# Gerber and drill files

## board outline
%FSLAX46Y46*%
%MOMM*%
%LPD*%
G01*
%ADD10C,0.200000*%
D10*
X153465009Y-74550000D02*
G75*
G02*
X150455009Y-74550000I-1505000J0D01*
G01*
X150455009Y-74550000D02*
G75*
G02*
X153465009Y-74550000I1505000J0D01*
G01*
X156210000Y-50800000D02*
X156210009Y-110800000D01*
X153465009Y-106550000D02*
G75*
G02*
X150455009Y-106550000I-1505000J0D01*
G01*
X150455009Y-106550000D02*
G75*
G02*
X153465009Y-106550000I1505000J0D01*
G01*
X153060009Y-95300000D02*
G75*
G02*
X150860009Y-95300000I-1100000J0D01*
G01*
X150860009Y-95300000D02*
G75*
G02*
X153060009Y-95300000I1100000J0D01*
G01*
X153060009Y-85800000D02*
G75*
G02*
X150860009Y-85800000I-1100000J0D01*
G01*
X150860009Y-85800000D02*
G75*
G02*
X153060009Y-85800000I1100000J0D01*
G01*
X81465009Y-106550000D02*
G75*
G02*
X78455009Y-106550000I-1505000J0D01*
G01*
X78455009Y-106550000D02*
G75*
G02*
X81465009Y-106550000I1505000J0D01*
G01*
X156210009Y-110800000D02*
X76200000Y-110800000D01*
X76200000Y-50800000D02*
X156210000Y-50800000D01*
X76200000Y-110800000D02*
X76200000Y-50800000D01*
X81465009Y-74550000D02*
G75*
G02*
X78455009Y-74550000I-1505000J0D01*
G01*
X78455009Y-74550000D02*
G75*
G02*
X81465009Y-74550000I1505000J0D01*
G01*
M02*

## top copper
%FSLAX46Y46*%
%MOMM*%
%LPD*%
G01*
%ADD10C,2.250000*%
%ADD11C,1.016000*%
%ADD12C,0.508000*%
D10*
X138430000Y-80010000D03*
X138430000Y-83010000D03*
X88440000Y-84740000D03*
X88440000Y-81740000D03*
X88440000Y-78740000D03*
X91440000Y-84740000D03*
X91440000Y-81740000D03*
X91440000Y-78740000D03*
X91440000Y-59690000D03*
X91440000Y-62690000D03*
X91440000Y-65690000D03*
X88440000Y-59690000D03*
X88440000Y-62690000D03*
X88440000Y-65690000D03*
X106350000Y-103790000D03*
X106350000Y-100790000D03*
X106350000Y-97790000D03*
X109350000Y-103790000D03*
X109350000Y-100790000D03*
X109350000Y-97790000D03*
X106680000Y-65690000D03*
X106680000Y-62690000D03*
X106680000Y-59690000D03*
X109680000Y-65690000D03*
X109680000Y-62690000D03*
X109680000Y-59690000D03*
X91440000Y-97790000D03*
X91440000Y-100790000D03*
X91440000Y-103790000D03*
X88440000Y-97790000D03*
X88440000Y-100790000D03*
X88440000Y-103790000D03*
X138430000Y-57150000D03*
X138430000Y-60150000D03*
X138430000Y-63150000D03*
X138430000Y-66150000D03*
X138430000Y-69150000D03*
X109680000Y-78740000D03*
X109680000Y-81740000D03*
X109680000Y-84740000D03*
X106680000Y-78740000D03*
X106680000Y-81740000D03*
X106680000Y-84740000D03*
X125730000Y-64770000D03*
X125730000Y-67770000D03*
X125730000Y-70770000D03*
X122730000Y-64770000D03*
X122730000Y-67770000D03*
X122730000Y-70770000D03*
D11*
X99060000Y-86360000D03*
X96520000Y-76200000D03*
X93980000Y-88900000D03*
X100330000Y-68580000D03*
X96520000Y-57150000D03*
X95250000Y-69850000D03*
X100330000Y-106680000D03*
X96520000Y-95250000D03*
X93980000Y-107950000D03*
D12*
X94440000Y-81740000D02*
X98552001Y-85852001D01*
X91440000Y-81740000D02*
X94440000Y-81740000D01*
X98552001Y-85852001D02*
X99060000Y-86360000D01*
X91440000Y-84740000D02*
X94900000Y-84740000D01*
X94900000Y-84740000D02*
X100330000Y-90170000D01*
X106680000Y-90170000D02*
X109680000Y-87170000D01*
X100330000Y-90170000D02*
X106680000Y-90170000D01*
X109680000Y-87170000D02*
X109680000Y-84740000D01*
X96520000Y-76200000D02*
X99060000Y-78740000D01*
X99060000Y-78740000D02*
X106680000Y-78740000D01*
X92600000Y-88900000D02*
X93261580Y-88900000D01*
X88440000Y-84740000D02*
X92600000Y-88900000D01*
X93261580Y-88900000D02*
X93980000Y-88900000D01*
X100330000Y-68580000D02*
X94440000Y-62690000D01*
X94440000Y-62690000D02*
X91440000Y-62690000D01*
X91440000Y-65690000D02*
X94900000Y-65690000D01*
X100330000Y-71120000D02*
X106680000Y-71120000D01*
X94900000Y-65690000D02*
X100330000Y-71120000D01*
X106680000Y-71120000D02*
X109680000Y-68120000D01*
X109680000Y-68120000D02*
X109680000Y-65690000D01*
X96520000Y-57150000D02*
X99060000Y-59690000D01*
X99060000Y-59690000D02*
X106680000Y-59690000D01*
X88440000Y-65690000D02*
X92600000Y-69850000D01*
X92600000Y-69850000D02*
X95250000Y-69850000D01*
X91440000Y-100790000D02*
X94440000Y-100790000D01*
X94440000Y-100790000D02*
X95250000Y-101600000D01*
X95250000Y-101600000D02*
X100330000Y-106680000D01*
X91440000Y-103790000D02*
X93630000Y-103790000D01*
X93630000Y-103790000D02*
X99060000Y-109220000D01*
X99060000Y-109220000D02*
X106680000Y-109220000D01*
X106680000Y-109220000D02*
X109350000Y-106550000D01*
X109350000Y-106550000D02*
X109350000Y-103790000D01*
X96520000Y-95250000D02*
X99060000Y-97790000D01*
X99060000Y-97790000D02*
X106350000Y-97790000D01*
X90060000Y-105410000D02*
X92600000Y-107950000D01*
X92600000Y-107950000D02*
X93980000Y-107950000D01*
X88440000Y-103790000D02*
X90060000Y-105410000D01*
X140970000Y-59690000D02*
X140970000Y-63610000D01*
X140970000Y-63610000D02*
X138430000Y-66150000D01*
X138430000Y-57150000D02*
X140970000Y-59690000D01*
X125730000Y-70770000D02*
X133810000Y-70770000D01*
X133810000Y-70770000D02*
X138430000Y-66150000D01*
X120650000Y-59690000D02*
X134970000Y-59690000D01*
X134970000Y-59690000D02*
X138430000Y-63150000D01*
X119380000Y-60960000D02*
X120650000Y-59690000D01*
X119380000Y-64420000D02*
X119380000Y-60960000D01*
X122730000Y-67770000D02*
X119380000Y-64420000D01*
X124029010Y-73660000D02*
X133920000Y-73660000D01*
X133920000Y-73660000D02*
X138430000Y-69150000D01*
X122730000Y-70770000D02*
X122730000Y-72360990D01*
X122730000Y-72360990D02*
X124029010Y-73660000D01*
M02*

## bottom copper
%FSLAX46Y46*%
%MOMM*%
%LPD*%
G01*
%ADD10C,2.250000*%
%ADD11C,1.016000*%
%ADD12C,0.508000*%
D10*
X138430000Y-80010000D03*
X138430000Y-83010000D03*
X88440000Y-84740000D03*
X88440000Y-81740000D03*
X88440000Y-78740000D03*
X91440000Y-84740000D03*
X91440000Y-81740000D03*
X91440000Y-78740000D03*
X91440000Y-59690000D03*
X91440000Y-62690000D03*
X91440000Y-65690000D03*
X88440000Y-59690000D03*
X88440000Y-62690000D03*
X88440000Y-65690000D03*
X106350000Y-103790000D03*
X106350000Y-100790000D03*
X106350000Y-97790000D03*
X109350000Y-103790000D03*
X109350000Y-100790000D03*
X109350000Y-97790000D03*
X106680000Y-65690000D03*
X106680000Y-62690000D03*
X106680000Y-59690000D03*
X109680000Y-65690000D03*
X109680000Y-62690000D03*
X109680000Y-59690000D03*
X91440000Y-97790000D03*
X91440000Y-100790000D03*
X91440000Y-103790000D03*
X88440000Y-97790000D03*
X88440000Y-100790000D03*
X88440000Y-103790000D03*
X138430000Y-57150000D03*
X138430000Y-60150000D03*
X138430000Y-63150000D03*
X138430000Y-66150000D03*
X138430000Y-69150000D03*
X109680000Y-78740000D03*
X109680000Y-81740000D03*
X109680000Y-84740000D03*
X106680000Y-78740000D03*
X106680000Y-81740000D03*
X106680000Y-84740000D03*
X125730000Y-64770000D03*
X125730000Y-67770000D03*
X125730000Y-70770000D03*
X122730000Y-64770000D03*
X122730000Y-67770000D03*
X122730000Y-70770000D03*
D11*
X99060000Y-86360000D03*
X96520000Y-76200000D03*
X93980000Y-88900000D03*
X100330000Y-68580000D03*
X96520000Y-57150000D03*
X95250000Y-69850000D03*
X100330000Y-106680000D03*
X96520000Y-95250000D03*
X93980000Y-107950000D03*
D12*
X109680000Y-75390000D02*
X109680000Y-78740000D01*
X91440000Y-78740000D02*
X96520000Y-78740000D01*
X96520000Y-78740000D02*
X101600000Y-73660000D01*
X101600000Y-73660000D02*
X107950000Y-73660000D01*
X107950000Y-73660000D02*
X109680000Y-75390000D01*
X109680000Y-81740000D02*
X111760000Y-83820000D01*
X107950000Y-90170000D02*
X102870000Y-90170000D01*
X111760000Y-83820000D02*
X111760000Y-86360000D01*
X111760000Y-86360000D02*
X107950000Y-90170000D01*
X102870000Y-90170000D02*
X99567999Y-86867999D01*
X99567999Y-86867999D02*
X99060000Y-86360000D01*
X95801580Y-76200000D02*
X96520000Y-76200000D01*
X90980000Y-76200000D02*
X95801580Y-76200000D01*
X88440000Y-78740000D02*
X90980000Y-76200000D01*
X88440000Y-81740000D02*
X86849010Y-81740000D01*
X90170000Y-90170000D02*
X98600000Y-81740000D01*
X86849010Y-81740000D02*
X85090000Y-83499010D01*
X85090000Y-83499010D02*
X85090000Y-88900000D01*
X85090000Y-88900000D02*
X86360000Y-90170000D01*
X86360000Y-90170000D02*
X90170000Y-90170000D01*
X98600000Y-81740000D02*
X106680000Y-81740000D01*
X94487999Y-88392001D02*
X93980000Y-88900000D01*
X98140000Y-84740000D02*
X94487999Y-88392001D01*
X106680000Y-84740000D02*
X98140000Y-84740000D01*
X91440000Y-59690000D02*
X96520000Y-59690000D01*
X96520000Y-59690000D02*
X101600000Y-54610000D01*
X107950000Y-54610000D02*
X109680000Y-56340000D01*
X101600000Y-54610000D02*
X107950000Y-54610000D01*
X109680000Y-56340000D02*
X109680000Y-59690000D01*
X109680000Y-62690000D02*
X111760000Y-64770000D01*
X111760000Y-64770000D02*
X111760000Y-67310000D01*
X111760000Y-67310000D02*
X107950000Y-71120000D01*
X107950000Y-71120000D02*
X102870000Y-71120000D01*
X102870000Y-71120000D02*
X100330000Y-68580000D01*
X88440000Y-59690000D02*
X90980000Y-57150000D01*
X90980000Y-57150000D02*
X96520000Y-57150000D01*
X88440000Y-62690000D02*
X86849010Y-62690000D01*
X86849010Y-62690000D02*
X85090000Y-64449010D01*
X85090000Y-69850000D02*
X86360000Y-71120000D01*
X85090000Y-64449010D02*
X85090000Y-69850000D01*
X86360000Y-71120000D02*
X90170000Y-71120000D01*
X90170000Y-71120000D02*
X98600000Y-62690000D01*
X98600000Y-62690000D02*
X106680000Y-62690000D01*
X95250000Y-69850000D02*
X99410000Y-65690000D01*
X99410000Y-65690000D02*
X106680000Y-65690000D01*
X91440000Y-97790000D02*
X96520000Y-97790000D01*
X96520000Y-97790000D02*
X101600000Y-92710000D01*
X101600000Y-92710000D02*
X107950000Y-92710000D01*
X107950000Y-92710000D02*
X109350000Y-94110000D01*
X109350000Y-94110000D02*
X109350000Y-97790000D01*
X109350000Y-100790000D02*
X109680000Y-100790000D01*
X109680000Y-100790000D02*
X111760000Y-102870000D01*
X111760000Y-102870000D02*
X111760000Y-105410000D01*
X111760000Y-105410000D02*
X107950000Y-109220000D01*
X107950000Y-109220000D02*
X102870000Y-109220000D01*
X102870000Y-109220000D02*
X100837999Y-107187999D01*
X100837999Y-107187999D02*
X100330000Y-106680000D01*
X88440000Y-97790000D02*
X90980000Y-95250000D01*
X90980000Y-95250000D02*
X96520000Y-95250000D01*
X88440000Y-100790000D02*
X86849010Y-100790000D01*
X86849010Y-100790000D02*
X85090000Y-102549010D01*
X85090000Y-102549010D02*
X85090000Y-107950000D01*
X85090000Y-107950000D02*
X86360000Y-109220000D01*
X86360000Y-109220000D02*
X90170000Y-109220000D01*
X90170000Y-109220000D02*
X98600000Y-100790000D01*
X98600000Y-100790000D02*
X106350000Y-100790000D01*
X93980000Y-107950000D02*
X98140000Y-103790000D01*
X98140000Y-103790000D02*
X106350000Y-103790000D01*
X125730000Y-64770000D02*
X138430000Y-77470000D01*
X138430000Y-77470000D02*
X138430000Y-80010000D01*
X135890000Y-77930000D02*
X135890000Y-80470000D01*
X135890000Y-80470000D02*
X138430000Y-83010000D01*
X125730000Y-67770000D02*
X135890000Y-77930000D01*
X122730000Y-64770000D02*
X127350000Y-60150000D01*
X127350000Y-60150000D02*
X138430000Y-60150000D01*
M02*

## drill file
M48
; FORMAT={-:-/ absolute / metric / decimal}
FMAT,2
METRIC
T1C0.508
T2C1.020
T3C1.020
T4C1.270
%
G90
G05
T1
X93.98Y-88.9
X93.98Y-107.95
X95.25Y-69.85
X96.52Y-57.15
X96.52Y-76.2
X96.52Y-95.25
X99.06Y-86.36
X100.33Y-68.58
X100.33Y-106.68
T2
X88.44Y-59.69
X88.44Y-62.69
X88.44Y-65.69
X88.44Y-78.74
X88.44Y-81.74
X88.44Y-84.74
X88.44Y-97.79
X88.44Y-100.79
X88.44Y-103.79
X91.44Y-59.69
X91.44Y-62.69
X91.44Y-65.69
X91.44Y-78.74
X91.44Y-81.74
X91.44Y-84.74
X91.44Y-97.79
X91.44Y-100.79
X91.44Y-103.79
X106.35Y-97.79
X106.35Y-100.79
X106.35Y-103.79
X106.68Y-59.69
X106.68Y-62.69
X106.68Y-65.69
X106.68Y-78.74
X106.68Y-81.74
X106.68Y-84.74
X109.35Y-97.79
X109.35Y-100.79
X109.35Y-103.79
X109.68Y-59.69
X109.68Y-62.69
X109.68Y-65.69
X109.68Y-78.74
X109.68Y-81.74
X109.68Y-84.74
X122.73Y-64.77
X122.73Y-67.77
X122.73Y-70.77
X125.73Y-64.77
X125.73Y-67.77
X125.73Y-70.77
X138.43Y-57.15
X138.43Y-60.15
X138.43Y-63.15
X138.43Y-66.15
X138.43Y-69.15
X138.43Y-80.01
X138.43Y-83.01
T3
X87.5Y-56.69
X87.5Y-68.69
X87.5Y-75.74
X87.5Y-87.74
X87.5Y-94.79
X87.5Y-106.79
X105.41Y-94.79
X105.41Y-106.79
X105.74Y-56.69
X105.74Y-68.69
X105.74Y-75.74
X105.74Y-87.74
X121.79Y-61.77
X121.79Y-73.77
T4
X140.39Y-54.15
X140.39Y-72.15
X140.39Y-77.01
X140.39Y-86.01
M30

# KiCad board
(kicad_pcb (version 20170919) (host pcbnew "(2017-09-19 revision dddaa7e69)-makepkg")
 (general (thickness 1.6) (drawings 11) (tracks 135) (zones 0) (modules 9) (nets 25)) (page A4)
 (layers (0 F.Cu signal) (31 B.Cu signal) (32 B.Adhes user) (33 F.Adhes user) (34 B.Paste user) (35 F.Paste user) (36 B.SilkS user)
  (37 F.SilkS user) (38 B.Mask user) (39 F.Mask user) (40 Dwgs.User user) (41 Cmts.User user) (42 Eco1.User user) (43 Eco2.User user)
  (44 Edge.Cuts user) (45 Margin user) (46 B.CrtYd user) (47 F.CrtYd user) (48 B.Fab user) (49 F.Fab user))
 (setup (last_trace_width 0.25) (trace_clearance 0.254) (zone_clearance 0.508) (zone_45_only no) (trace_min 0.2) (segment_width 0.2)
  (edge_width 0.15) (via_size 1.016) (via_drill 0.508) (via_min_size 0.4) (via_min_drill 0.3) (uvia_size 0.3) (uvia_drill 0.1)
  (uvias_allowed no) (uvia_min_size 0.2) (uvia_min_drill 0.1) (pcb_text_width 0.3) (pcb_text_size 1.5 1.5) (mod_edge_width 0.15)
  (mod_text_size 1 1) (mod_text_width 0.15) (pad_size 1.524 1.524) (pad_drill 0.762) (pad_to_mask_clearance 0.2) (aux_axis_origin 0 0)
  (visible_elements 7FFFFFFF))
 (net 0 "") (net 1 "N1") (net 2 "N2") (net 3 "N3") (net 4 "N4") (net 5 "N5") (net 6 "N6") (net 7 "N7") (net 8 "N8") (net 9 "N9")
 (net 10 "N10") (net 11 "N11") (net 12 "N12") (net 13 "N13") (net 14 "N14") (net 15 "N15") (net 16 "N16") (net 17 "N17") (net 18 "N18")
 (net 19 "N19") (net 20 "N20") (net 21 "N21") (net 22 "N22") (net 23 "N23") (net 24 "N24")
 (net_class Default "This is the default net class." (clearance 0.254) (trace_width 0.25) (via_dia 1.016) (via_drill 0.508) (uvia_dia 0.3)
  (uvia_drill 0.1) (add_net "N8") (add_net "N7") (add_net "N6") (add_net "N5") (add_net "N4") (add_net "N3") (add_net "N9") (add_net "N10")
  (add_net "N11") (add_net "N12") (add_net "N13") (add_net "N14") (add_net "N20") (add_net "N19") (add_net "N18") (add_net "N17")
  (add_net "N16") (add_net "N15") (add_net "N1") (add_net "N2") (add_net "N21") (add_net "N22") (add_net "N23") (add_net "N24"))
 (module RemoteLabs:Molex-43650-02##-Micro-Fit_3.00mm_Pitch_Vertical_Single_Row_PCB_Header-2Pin (layer F.Cu) (at 138.43 80.01 90)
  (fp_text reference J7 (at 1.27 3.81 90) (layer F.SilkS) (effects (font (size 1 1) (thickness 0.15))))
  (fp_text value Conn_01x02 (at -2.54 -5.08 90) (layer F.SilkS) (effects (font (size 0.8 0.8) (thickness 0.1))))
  (pad 1 thru_hole circle (at 0 0 90) (size 2.25 2.25) (drill 1.02) (layers *.Cu *.Mask F.SilkS) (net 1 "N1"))
  (pad 2 thru_hole circle (at -3 0 90) (size 2.25 2.25) (drill 1.02) (layers *.Cu *.Mask F.SilkS) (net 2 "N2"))
  (pad "" np_thru_hole circle (at 3 1.96 90) (size 1.27 1.27) (drill 1.27) (layers *.Cu *.Mask F.SilkS))
  (pad "" np_thru_hole circle (at -6 1.96 90) (size 1.27 1.27) (drill 1.27) (layers *.Cu *.Mask F.SilkS)))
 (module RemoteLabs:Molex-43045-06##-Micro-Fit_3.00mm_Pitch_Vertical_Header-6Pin (layer F.Cu) (at 91.44 78.74 90)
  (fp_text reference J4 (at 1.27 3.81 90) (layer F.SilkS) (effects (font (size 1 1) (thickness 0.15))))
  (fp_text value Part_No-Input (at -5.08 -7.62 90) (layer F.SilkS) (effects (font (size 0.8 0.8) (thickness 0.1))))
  (pad 6 thru_hole circle (at -6 -3 90) (size 2.25 2.25) (drill 1.02) (layers *.Cu *.Mask F.SilkS) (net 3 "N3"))
  (pad 5 thru_hole circle (at -3 -3 90) (size 2.25 2.25) (drill 1.02) (layers *.Cu *.Mask F.SilkS) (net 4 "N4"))
  (pad 4 thru_hole circle (at 0 -3 90) (size 2.25 2.25) (drill 1.02) (layers *.Cu *.Mask F.SilkS) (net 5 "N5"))
  (pad 3 thru_hole circle (at -6 0 90) (size 2.25 2.25) (drill 1.02) (layers *.Cu *.Mask F.SilkS) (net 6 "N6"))
  (pad 2 thru_hole circle (at -3 0 90) (size 2.25 2.25) (drill 1.02) (layers *.Cu *.Mask F.SilkS) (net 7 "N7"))
  (pad 1 thru_hole circle (at 0 0 90) (size 2.25 2.25) (drill 1.02) (layers *.Cu *.Mask F.SilkS) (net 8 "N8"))
  (pad "" np_thru_hole circle (at -9 -3.94 90) (size 1.02 1.02) (drill 1.02) (layers *.Cu *.Mask F.SilkS))
  (pad "" np_thru_hole circle (at 3 -3.94 90) (size 1.02 1.02) (drill 1.02) (layers *.Cu *.Mask F.SilkS)))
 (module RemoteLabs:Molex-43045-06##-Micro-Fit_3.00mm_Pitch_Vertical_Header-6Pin (layer F.Cu) (at 91.44 59.69 90)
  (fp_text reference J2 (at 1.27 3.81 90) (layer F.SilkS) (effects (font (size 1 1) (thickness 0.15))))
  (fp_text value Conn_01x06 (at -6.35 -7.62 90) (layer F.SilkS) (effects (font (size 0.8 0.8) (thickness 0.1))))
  (pad "" np_thru_hole circle (at 3 -3.94 90) (size 1.02 1.02) (drill 1.02) (layers *.Cu *.Mask F.SilkS))
  (pad "" np_thru_hole circle (at -9 -3.94 90) (size 1.02 1.02) (drill 1.02) (layers *.Cu *.Mask F.SilkS))
  (pad 1 thru_hole circle (at 0 0 90) (size 2.25 2.25) (drill 1.02) (layers *.Cu *.Mask F.SilkS) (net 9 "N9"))
  (pad 2 thru_hole circle (at -3 0 90) (size 2.25 2.25) (drill 1.02) (layers *.Cu *.Mask F.SilkS) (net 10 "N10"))
  (pad 3 thru_hole circle (at -6 0 90) (size 2.25 2.25) (drill 1.02) (layers *.Cu *.Mask F.SilkS) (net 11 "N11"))
  (pad 4 thru_hole circle (at 0 -3 90) (size 2.25 2.25) (drill 1.02) (layers *.Cu *.Mask F.SilkS) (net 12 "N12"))
  (pad 5 thru_hole circle (at -3 -3 90) (size 2.25 2.25) (drill 1.02) (layers *.Cu *.Mask F.SilkS) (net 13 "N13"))
  (pad 6 thru_hole circle (at -6 -3 90) (size 2.25 2.25) (drill 1.02) (layers *.Cu *.Mask F.SilkS) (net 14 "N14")))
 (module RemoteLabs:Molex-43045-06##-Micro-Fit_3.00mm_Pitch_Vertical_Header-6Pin (layer F.Cu) (at 109.35 97.79 90)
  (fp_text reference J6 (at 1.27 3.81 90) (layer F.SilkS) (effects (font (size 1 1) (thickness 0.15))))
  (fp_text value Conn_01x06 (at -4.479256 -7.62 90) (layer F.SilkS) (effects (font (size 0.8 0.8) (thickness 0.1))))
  (pad 6 thru_hole circle (at -6 -3 90) (size 2.25 2.25) (drill 1.02) (layers *.Cu *.Mask F.SilkS) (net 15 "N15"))
  (pad 5 thru_hole circle (at -3 -3 90) (size 2.25 2.25) (drill 1.02) (layers *.Cu *.Mask F.SilkS) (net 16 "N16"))
  (pad 4 thru_hole circle (at 0 -3 90) (size 2.25 2.25) (drill 1.02) (layers *.Cu *.Mask F.SilkS) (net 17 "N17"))
  (pad 3 thru_hole circle (at -6 0 90) (size 2.25 2.25) (drill 1.02) (layers *.Cu *.Mask F.SilkS) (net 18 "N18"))
  (pad 2 thru_hole circle (at -3 0 90) (size 2.25 2.25) (drill 1.02) (layers *.Cu *.Mask F.SilkS) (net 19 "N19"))
  (pad 1 thru_hole circle (at 0 0 90) (size 2.25 2.25) (drill 1.02) (layers *.Cu *.Mask F.SilkS) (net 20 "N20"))
  (pad "" np_thru_hole circle (at -9 -3.94 90) (size 1.02 1.02) (drill 1.02) (layers *.Cu *.Mask F.SilkS))
  (pad "" np_thru_hole circle (at 3 -3.94 90) (size 1.02 1.02) (drill 1.02) (layers *.Cu *.Mask F.SilkS)))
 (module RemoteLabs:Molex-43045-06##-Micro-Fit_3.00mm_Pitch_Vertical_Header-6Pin (layer F.Cu) (at 109.68 59.69 90)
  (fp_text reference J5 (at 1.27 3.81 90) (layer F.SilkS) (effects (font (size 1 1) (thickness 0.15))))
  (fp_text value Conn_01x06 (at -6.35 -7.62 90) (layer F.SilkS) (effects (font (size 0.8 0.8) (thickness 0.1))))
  (pad 6 thru_hole circle (at -6 -3 90) (size 2.25 2.25) (drill 1.02) (layers *.Cu *.Mask F.SilkS) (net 14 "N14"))
  (pad 5 thru_hole circle (at -3 -3 90) (size 2.25 2.25) (drill 1.02) (layers *.Cu *.Mask F.SilkS) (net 13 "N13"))
  (pad 4 thru_hole circle (at 0 -3 90) (size 2.25 2.25) (drill 1.02) (layers *.Cu *.Mask F.SilkS) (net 12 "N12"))
  (pad 3 thru_hole circle (at -6 0 90) (size 2.25 2.25) (drill 1.02) (layers *.Cu *.Mask F.SilkS) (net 11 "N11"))
  (pad 2 thru_hole circle (at -3 0 90) (size 2.25 2.25) (drill 1.02) (layers *.Cu *.Mask F.SilkS) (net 10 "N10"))
  (pad 1 thru_hole circle (at 0 0 90) (size 2.25 2.25) (drill 1.02) (layers *.Cu *.Mask F.SilkS) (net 9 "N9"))
  (pad "" np_thru_hole circle (at -9 -3.94 90) (size 1.02 1.02) (drill 1.02) (layers *.Cu *.Mask F.SilkS))
  (pad "" np_thru_hole circle (at 3 -3.94 90) (size 1.02 1.02) (drill 1.02) (layers *.Cu *.Mask F.SilkS)))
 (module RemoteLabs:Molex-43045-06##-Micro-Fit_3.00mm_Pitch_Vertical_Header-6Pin (layer F.Cu) (at 91.44 97.79 90)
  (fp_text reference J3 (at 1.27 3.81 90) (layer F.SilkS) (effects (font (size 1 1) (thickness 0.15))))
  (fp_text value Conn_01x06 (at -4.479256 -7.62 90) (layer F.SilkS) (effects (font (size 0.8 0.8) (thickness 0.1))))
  (pad "" np_thru_hole circle (at 3 -3.94 90) (size 1.02 1.02) (drill 1.02) (layers *.Cu *.Mask F.SilkS))
  (pad "" np_thru_hole circle (at -9 -3.94 90) (size 1.02 1.02) (drill 1.02) (layers *.Cu *.Mask F.SilkS))
  (pad 1 thru_hole circle (at 0 0 90) (size 2.25 2.25) (drill 1.02) (layers *.Cu *.Mask F.SilkS) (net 20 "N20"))
  (pad 2 thru_hole circle (at -3 0 90) (size 2.25 2.25) (drill 1.02) (layers *.Cu *.Mask F.SilkS) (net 19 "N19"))
  (pad 3 thru_hole circle (at -6 0 90) (size 2.25 2.25) (drill 1.02) (layers *.Cu *.Mask F.SilkS) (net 18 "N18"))
  (pad 4 thru_hole circle (at 0 -3 90) (size 2.25 2.25) (drill 1.02) (layers *.Cu *.Mask F.SilkS) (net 17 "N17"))
  (pad 5 thru_hole circle (at -3 -3 90) (size 2.25 2.25) (drill 1.02) (layers *.Cu *.Mask F.SilkS) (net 16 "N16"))
  (pad 6 thru_hole circle (at -6 -3 90) (size 2.25 2.25) (drill 1.02) (layers *.Cu *.Mask F.SilkS) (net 15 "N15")))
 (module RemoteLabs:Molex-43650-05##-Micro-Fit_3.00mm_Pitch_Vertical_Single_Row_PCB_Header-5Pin (layer F.Cu) (at 138.43 57.15 90)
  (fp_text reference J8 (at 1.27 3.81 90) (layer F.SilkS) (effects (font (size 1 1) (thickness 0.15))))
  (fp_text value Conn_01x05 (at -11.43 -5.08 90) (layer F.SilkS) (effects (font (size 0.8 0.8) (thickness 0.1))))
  (pad 1 thru_hole circle (at 0 0 90) (size 2.25 2.25) (drill 1.02) (layers *.Cu *.Mask F.SilkS) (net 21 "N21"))
  (pad 2 thru_hole circle (at -3 0 90) (size 2.25 2.25) (drill 1.02) (layers *.Cu *.Mask F.SilkS) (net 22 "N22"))
  (pad 3 thru_hole circle (at -6 0 90) (size 2.25 2.25) (drill 1.02) (layers *.Cu *.Mask F.SilkS) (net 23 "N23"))
  (pad 4 thru_hole circle (at -9 0 90) (size 2.25 2.25) (drill 1.02) (layers *.Cu *.Mask F.SilkS) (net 21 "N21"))
  (pad 5 thru_hole circle (at -12 0 90) (size 2.25 2.25) (drill 1.02) (layers *.Cu *.Mask F.SilkS) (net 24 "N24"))
  (pad "" np_thru_hole circle (at 3 1.96 90) (size 1.27 1.27) (drill 1.27) (layers *.Cu *.Mask F.SilkS))
  (pad "" np_thru_hole circle (at -15 1.96 90) (size 1.27 1.27) (drill 1.27) (layers *.Cu *.Mask F.SilkS)))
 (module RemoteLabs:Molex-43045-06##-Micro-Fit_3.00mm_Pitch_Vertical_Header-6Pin (layer F.Cu) (at 109.68 78.74 90)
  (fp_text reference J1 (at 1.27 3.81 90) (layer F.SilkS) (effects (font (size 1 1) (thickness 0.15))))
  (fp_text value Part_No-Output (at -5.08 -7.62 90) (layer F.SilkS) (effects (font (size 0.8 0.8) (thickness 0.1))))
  (pad "" np_thru_hole circle (at 3 -3.94 90) (size 1.02 1.02) (drill 1.02) (layers *.Cu *.Mask F.SilkS))
  (pad "" np_thru_hole circle (at -9 -3.94 90) (size 1.02 1.02) (drill 1.02) (layers *.Cu *.Mask F.SilkS))
  (pad 1 thru_hole circle (at 0 0 90) (size 2.25 2.25) (drill 1.02) (layers *.Cu *.Mask F.SilkS) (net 8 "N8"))
  (pad 2 thru_hole circle (at -3 0 90) (size 2.25 2.25) (drill 1.02) (layers *.Cu *.Mask F.SilkS) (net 7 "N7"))
  (pad 3 thru_hole circle (at -6 0 90) (size 2.25 2.25) (drill 1.02) (layers *.Cu *.Mask F.SilkS) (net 6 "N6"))
  (pad 4 thru_hole circle (at 0 -3 90) (size 2.25 2.25) (drill 1.02) (layers *.Cu *.Mask F.SilkS) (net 5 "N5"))
  (pad 5 thru_hole circle (at -3 -3 90) (size 2.25 2.25) (drill 1.02) (layers *.Cu *.Mask F.SilkS) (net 4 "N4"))
  (pad 6 thru_hole circle (at -6 -3 90) (size 2.25 2.25) (drill 1.02) (layers *.Cu *.Mask F.SilkS) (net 3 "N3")))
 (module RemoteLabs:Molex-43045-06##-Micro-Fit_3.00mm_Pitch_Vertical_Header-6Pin (layer F.Cu) (at 125.73 64.77 90)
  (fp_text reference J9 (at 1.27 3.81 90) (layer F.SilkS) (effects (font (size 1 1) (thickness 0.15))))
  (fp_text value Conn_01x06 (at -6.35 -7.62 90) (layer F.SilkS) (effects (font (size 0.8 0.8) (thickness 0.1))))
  (pad "" np_thru_hole circle (at 3 -3.94 90) (size 1.02 1.02) (drill 1.02) (layers *.Cu *.Mask F.SilkS))
  (pad "" np_thru_hole circle (at -9 -3.94 90) (size 1.02 1.02) (drill 1.02) (layers *.Cu *.Mask F.SilkS))
  (pad 1 thru_hole circle (at 0 0 90) (size 2.25 2.25) (drill 1.02) (layers *.Cu *.Mask F.SilkS) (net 1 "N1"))
  (pad 2 thru_hole circle (at -3 0 90) (size 2.25 2.25) (drill 1.02) (layers *.Cu *.Mask F.SilkS) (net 2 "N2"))
  (pad 3 thru_hole circle (at -6 0 90) (size 2.25 2.25) (drill 1.02) (layers *.Cu *.Mask F.SilkS) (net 21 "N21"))
  (pad 4 thru_hole circle (at 0 -3 90) (size 2.25 2.25) (drill 1.02) (layers *.Cu *.Mask F.SilkS) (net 22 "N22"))
  (pad 5 thru_hole circle (at -3 -3 90) (size 2.25 2.25) (drill 1.02) (layers *.Cu *.Mask F.SilkS) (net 23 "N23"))
  (pad 6 thru_hole circle (at -6 -3 90) (size 2.25 2.25) (drill 1.02) (layers *.Cu *.Mask F.SilkS) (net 24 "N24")))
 (gr_circle (center 151.960009 74.55) (end 153.465009 74.55) (layer Edge.Cuts) (width 0.2))
 (gr_line (start 156.21 50.8) (end 156.210009 110.8) (layer Edge.Cuts) (width 0.2))
 (gr_circle (center 151.960009 106.55) (end 153.465009 106.55) (layer Edge.Cuts) (width 0.2))
 (gr_circle (center 151.960009 95.3) (end 153.060009 95.3) (layer Edge.Cuts) (width 0.2))
 (gr_circle (center 151.960009 85.8) (end 153.060009 85.8) (layer Edge.Cuts) (width 0.2))
 (gr_circle (center 79.960009 106.55) (end 81.465009 106.55) (layer Edge.Cuts) (width 0.2))
 (gr_line (start 156.210009 110.8) (end 76.2 110.8) (layer Edge.Cuts) (width 0.2))
 (gr_line (start 76.2 50.8) (end 156.21 50.8) (layer Edge.Cuts) (width 0.2))
 (gr_line (start 76.2 110.8) (end 76.2 50.8) (layer Edge.Cuts) (width 0.2))
 (gr_circle (center 79.960009 74.55) (end 81.465009 74.55) (layer Edge.Cuts) (width 0.2))
 (segment (start 109.68 75.39) (end 109.68 78.74) (width 0.508) (layer B.Cu) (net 8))
 (segment (start 91.44 78.74) (end 96.52 78.74) (width 0.508) (layer B.Cu) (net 8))
 (segment (start 96.52 78.74) (end 101.6 73.66) (width 0.508) (layer B.Cu) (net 8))
 (segment (start 101.6 73.66) (end 107.95 73.66) (width 0.508) (layer B.Cu) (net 8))
 (segment (start 107.95 73.66) (end 109.68 75.39) (width 0.508) (layer B.Cu) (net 8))
 (segment (start 109.68 81.74) (end 111.76 83.82) (width 0.508) (layer B.Cu) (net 7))
 (segment (start 107.95 90.17) (end 102.87 90.17) (width 0.508) (layer B.Cu) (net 7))
 (segment (start 111.76 83.82) (end 111.76 86.36) (width 0.508) (layer B.Cu) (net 7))
 (segment (start 111.76 86.36) (end 107.95 90.17) (width 0.508) (layer B.Cu) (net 7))
 (segment (start 102.87 90.17) (end 99.567999 86.867999) (width 0.508) (layer B.Cu) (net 7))
 (segment (start 99.567999 86.867999) (end 99.06 86.36) (width 0.508) (layer B.Cu) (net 7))
 (segment (start 94.44 81.74) (end 98.552001 85.852001) (width 0.508) (layer F.Cu) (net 7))
 (segment (start 91.44 81.74) (end 94.44 81.74) (width 0.508) (layer F.Cu) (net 7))
 (segment (start 98.552001 85.852001) (end 99.06 86.36) (width 0.508) (layer F.Cu) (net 7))
 (via (at 99.06 86.36) (size 1.016) (drill 0.508) (layers F.Cu B.Cu) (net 7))
 (segment (start 91.44 84.74) (end 94.9 84.74) (width 0.508) (layer F.Cu) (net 6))
 (segment (start 94.9 84.74) (end 100.33 90.17) (width 0.508) (layer F.Cu) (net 6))
 (segment (start 106.68 90.17) (end 109.68 87.17) (width 0.508) (layer F.Cu) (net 6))
 (segment (start 100.33 90.17) (end 106.68 90.17) (width 0.508) (layer F.Cu) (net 6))
 (segment (start 109.68 87.17) (end 109.68 84.74) (width 0.508) (layer F.Cu) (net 6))
 (segment (start 96.52 76.2) (end 99.06 78.74) (width 0.508) (layer F.Cu) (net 5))
 (segment (start 99.06 78.74) (end 106.68 78.74) (width 0.508) (layer F.Cu) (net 5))
 (segment (start 95.80158 76.2) (end 96.52 76.2) (width 0.508) (layer B.Cu) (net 5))
 (segment (start 90.98 76.2) (end 95.80158 76.2) (width 0.508) (layer B.Cu) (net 5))
 (segment (start 88.44 78.74) (end 90.98 76.2) (width 0.508) (layer B.Cu) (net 5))
 (via (at 96.52 76.2) (size 1.016) (drill 0.508) (layers F.Cu B.Cu) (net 5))
 (segment (start 88.44 81.74) (end 86.84901 81.74) (width 0.508) (layer B.Cu) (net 4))
 (segment (start 90.17 90.17) (end 98.6 81.74) (width 0.508) (layer B.Cu) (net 4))
 (segment (start 86.84901 81.74) (end 85.09 83.49901) (width 0.508) (layer B.Cu) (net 4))
 (segment (start 85.09 83.49901) (end 85.09 88.9) (width 0.508) (layer B.Cu) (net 4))
 (segment (start 85.09 88.9) (end 86.36 90.17) (width 0.508) (layer B.Cu) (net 4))
 (segment (start 86.36 90.17) (end 90.17 90.17) (width 0.508) (layer B.Cu) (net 4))
 (segment (start 98.6 81.74) (end 106.68 81.74) (width 0.508) (layer B.Cu) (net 4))
 (segment (start 92.6 88.9) (end 93.26158 88.9) (width 0.508) (layer F.Cu) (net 3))
 (segment (start 88.44 84.74) (end 92.6 88.9) (width 0.508) (layer F.Cu) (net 3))
 (segment (start 93.26158 88.9) (end 93.98 88.9) (width 0.508) (layer F.Cu) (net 3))
 (segment (start 94.487999 88.392001) (end 93.98 88.9) (width 0.508) (layer B.Cu) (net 3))
 (segment (start 98.14 84.74) (end 94.487999 88.392001) (width 0.508) (layer B.Cu) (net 3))
 (segment (start 106.68 84.74) (end 98.14 84.74) (width 0.508) (layer B.Cu) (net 3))
 (via (at 93.98 88.9) (size 1.016) (drill 0.508) (layers F.Cu B.Cu) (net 3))
 (segment (start 91.44 59.69) (end 96.52 59.69) (width 0.508) (layer B.Cu) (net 9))
 (segment (start 96.52 59.69) (end 101.6 54.61) (width 0.508) (layer B.Cu) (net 9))
 (segment (start 107.95 54.61) (end 109.68 56.34) (width 0.508) (layer B.Cu) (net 9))
 (segment (start 101.6 54.61) (end 107.95 54.61) (width 0.508) (layer B.Cu) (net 9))
 (segment (start 109.68 56.34) (end 109.68 59.69) (width 0.508) (layer B.Cu) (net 9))
 (segment (start 109.68 62.69) (end 111.76 64.77) (width 0.508) (layer B.Cu) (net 10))
 (segment (start 111.76 64.77) (end 111.76 67.31) (width 0.508) (layer B.Cu) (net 10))
 (segment (start 111.76 67.31) (end 107.95 71.12) (width 0.508) (layer B.Cu) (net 10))
 (segment (start 107.95 71.12) (end 102.87 71.12) (width 0.508) (layer B.Cu) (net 10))
 (segment (start 102.87 71.12) (end 100.33 68.58) (width 0.508) (layer B.Cu) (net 10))
 (segment (start 100.33 68.58) (end 94.44 62.69) (width 0.508) (layer F.Cu) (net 10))
 (segment (start 94.44 62.69) (end 91.44 62.69) (width 0.508) (layer F.Cu) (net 10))
 (via (at 100.33 68.58) (size 1.016) (drill 0.508) (layers F.Cu B.Cu) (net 10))
 (segment (start 91.44 65.69) (end 94.9 65.69) (width 0.508) (layer F.Cu) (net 11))
 (segment (start 100.33 71.12) (end 106.68 71.12) (width 0.508) (layer F.Cu) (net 11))
 (segment (start 94.9 65.69) (end 100.33 71.12) (width 0.508) (layer F.Cu) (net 11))
 (segment (start 106.68 71.12) (end 109.68 68.12) (width 0.508) (layer F.Cu) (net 11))
 (segment (start 109.68 68.12) (end 109.68 65.69) (width 0.508) (layer F.Cu) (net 11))
 (segment (start 96.52 57.15) (end 99.06 59.69) (width 0.508) (layer F.Cu) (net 12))
 (segment (start 99.06 59.69) (end 106.68 59.69) (width 0.508) (layer F.Cu) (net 12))
 (segment (start 88.44 59.69) (end 90.98 57.15) (width 0.508) (layer B.Cu) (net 12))
 (segment (start 90.98 57.15) (end 96.52 57.15) (width 0.508) (layer B.Cu) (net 12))
 (via (at 96.52 57.15) (size 1.016) (drill 0.508) (layers F.Cu B.Cu) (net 12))
 (segment (start 88.44 62.69) (end 86.84901 62.69) (width 0.508) (layer B.Cu) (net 13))
 (segment (start 86.84901 62.69) (end 85.09 64.44901) (width 0.508) (layer B.Cu) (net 13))
 (segment (start 85.09 69.85) (end 86.36 71.12) (width 0.508) (layer B.Cu) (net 13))
 (segment (start 85.09 64.44901) (end 85.09 69.85) (width 0.508) (layer B.Cu) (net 13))
 (segment (start 86.36 71.12) (end 90.17 71.12) (width 0.508) (layer B.Cu) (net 13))
 (segment (start 90.17 71.12) (end 98.6 62.69) (width 0.508) (layer B.Cu) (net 13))
 (segment (start 98.6 62.69) (end 106.68 62.69) (width 0.508) (layer B.Cu) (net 13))
 (segment (start 95.25 69.85) (end 99.41 65.69) (width 0.508) (layer B.Cu) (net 14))
 (segment (start 99.41 65.69) (end 106.68 65.69) (width 0.508) (layer B.Cu) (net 14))
 (segment (start 88.44 65.69) (end 92.6 69.85) (width 0.508) (layer F.Cu) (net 14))
 (segment (start 92.6 69.85) (end 95.25 69.85) (width 0.508) (layer F.Cu) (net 14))
 (via (at 95.25 69.85) (size 1.016) (drill 0.508) (layers F.Cu B.Cu) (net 14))
 (segment (start 91.44 97.79) (end 96.52 97.79) (width 0.508) (layer B.Cu) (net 20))
 (segment (start 96.52 97.79) (end 101.6 92.71) (width 0.508) (layer B.Cu) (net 20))
 (segment (start 101.6 92.71) (end 107.95 92.71) (width 0.508) (layer B.Cu) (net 20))
 (segment (start 107.95 92.71) (end 109.35 94.11) (width 0.508) (layer B.Cu) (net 20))
 (segment (start 109.35 94.11) (end 109.35 97.79) (width 0.508) (layer B.Cu) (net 20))
 (segment (start 109.35 100.79) (end 109.68 100.79) (width 0.508) (layer B.Cu) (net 19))
 (segment (start 109.68 100.79) (end 111.76 102.87) (width 0.508) (layer B.Cu) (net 19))
 (segment (start 111.76 102.87) (end 111.76 105.41) (width 0.508) (layer B.Cu) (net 19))
 (segment (start 111.76 105.41) (end 107.95 109.22) (width 0.508) (layer B.Cu) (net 19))
 (segment (start 107.95 109.22) (end 102.87 109.22) (width 0.508) (layer B.Cu) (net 19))
 (segment (start 102.87 109.22) (end 100.837999 107.187999) (width 0.508) (layer B.Cu) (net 19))
 (segment (start 100.837999 107.187999) (end 100.33 106.68) (width 0.508) (layer B.Cu) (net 19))
 (segment (start 91.44 100.79) (end 94.44 100.79) (width 0.508) (layer F.Cu) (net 19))
 (segment (start 94.44 100.79) (end 95.25 101.6) (width 0.508) (layer F.Cu) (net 19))
 (segment (start 95.25 101.6) (end 100.33 106.68) (width 0.508) (layer F.Cu) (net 19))
 (via (at 100.33 106.68) (size 1.016) (drill 0.508) (layers F.Cu B.Cu) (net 19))
 (segment (start 91.44 103.79) (end 93.63 103.79) (width 0.508) (layer F.Cu) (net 18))
 (segment (start 93.63 103.79) (end 99.06 109.22) (width 0.508) (layer F.Cu) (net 18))
 (segment (start 99.06 109.22) (end 106.68 109.22) (width 0.508) (layer F.Cu) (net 18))
 (segment (start 106.68 109.22) (end 109.35 106.55) (width 0.508) (layer F.Cu) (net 18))
 (segment (start 109.35 106.55) (end 109.35 103.79) (width 0.508) (layer F.Cu) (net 18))
 (segment (start 96.52 95.25) (end 99.06 97.79) (width 0.508) (layer F.Cu) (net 17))
 (segment (start 99.06 97.79) (end 106.35 97.79) (width 0.508) (layer F.Cu) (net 17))
 (segment (start 88.44 97.79) (end 90.98 95.25) (width 0.508) (layer B.Cu) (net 17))
 (segment (start 90.98 95.25) (end 96.52 95.25) (width 0.508) (layer B.Cu) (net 17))
 (via (at 96.52 95.25) (size 1.016) (drill 0.508) (layers F.Cu B.Cu) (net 17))
 (segment (start 88.44 100.79) (end 86.84901 100.79) (width 0.508) (layer B.Cu) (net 16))
 (segment (start 86.84901 100.79) (end 85.09 102.54901) (width 0.508) (layer B.Cu) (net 16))
 (segment (start 85.09 102.54901) (end 85.09 107.95) (width 0.508) (layer B.Cu) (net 16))
 (segment (start 85.09 107.95) (end 86.36 109.22) (width 0.508) (layer B.Cu) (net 16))
 (segment (start 86.36 109.22) (end 90.17 109.22) (width 0.508) (layer B.Cu) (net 16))
 (segment (start 90.17 109.22) (end 98.6 100.79) (width 0.508) (layer B.Cu) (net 16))
 (segment (start 98.6 100.79) (end 106.35 100.79) (width 0.508) (layer B.Cu) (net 16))
 (segment (start 93.98 107.95) (end 98.14 103.79) (width 0.508) (layer B.Cu) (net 15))
 (segment (start 98.14 103.79) (end 106.35 103.79) (width 0.508) (layer B.Cu) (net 15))
 (segment (start 90.06 105.41) (end 92.6 107.95) (width 0.508) (layer F.Cu) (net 15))
 (segment (start 92.6 107.95) (end 93.98 107.95) (width 0.508) (layer F.Cu) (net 15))
 (via (at 93.98 107.95) (size 1.016) (drill 0.508) (layers F.Cu B.Cu) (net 15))
 (segment (start 88.44 103.79) (end 90.06 105.41) (width 0.508) (layer F.Cu) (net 15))
 (segment (start 125.73 64.77) (end 138.43 77.47) (width 0.508) (layer B.Cu) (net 1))
 (segment (start 138.43 77.47) (end 138.43 80.01) (width 0.508) (layer B.Cu) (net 1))
 (segment (start 135.89 77.93) (end 135.89 80.47) (width 0.508) (layer B.Cu) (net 2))
 (segment (start 135.89 80.47) (end 138.43 83.01) (width 0.508) (layer B.Cu) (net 2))
 (segment (start 125.73 67.77) (end 135.89 77.93) (width 0.508) (layer B.Cu) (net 2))
 (segment (start 140.97 59.69) (end 140.97 63.61) (width 0.508) (layer F.Cu) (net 21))
 (segment (start 140.97 63.61) (end 138.43 66.15) (width 0.508) (layer F.Cu) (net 21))
 (segment (start 138.43 57.15) (end 140.97 59.69) (width 0.508) (layer F.Cu) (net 21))
 (segment (start 125.73 70.77) (end 133.81 70.77) (width 0.508) (layer F.Cu) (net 21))
 (segment (start 133.81 70.77) (end 138.43 66.15) (width 0.508) (layer F.Cu) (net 21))
 (segment (start 122.73 64.77) (end 127.35 60.15) (width 0.508) (layer B.Cu) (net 22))
 (segment (start 127.35 60.15) (end 138.43 60.15) (width 0.508) (layer B.Cu) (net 22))
 (segment (start 120.65 59.69) (end 134.97 59.69) (width 0.508) (layer F.Cu) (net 23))
 (segment (start 134.97 59.69) (end 138.43 63.15) (width 0.508) (layer F.Cu) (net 23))
 (segment (start 119.38 60.96) (end 120.65 59.69) (width 0.508) (layer F.Cu) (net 23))
 (segment (start 119.38 64.42) (end 119.38 60.96) (width 0.508) (layer F.Cu) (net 23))
 (segment (start 122.73 67.77) (end 119.38 64.42) (width 0.508) (layer F.Cu) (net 23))
 (segment (start 124.02901 73.66) (end 133.92 73.66) (width 0.508) (layer F.Cu) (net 24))
 (segment (start 133.92 73.66) (end 138.43 69.15) (width 0.508) (layer F.Cu) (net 24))
 (segment (start 122.73 70.77) (end 122.73 72.36099) (width 0.508) (layer F.Cu) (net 24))
 (segment (start 122.73 72.36099) (end 124.02901 73.66) (width 0.508) (layer F.Cu) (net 24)))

